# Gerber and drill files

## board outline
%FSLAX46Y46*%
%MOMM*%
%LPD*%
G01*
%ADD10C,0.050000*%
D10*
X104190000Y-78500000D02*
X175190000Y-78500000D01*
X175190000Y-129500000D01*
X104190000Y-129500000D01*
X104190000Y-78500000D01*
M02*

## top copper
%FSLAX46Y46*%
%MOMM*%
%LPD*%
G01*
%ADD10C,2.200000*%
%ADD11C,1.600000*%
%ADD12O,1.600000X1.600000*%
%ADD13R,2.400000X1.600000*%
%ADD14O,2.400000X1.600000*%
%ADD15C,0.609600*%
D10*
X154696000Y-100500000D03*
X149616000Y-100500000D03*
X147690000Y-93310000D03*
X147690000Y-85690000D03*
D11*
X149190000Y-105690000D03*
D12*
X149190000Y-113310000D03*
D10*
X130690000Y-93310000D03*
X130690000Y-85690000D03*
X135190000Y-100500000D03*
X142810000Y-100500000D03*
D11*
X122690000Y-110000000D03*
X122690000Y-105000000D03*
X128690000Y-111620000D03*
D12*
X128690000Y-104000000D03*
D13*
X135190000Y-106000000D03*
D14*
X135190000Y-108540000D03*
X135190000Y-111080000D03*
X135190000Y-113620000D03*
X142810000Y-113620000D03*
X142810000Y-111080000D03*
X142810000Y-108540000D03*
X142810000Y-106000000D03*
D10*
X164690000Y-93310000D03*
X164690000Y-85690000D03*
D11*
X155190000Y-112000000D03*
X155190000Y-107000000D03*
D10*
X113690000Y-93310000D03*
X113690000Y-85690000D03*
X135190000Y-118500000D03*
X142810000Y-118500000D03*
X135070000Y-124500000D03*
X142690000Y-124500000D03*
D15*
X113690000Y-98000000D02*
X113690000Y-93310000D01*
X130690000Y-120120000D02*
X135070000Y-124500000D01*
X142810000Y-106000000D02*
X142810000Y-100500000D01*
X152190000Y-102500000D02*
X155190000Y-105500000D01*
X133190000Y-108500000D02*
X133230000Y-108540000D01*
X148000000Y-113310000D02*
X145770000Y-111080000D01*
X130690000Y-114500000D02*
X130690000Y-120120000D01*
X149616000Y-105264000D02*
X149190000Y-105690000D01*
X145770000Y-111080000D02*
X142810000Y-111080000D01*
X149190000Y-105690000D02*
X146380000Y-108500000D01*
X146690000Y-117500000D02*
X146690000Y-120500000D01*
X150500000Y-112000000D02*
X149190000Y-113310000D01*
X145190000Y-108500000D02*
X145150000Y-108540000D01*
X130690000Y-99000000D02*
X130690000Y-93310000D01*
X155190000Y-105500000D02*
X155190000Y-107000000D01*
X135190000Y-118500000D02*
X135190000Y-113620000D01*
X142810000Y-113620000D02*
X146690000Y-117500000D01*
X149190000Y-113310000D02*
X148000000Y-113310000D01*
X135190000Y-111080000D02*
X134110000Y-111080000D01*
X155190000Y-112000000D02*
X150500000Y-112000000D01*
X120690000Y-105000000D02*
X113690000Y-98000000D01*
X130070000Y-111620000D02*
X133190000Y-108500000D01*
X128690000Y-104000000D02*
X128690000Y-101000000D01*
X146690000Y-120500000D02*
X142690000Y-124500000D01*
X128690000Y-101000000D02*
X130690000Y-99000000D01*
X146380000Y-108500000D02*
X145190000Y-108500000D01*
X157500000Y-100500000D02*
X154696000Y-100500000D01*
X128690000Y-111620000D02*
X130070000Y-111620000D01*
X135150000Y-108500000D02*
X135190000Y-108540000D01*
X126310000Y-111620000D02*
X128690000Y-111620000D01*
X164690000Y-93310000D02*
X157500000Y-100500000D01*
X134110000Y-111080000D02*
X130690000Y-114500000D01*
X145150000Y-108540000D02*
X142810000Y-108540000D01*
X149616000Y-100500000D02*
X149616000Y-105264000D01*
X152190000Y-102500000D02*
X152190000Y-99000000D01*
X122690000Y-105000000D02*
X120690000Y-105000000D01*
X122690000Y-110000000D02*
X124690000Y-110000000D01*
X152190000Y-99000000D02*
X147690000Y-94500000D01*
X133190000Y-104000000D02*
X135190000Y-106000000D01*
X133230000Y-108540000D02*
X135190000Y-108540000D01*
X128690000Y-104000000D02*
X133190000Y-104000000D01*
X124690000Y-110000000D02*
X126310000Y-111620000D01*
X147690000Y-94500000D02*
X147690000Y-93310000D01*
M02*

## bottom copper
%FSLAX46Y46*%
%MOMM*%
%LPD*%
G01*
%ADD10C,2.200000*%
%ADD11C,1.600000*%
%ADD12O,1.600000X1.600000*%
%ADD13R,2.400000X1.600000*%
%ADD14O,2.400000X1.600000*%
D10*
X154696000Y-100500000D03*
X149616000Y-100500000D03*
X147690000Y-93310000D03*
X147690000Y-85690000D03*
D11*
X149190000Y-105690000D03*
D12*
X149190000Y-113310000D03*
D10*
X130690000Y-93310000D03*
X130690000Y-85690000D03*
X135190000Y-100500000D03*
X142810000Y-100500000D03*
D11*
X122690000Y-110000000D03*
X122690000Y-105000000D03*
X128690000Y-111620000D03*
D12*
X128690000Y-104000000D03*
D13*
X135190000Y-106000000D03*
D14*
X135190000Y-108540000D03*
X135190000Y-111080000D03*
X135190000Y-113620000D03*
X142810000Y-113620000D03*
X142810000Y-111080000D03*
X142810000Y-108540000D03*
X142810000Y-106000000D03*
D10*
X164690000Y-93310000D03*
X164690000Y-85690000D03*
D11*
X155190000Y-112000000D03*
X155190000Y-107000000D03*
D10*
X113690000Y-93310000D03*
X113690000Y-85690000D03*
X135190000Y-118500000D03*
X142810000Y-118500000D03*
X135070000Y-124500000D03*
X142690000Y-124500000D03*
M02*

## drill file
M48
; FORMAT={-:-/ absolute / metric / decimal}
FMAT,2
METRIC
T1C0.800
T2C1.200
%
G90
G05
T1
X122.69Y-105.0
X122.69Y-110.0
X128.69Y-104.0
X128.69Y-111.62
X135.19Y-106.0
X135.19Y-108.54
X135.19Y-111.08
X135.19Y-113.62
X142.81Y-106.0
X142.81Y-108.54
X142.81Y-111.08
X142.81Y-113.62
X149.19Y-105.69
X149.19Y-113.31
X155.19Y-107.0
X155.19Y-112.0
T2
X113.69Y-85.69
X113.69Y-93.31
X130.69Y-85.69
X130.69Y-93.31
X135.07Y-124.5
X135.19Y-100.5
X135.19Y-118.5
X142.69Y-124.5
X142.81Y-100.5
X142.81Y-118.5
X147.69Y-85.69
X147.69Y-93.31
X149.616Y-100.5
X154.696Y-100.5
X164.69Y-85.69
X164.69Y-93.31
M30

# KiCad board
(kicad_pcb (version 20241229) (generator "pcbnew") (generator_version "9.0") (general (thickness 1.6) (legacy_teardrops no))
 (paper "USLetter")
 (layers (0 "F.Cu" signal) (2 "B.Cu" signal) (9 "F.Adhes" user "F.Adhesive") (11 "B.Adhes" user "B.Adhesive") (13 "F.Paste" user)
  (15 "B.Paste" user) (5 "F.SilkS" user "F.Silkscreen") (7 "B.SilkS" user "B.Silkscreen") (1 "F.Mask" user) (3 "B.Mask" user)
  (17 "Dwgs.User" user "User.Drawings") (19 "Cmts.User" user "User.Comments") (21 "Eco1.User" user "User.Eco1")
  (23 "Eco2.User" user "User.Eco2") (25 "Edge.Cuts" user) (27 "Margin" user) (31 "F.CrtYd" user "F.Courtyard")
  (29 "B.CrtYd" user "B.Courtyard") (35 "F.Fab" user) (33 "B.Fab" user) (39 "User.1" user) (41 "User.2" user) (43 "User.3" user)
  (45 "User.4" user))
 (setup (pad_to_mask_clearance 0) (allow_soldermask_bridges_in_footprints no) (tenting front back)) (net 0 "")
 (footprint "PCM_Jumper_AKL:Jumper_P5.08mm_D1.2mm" (layer "F.Cu") (at 154.696 100.5 180)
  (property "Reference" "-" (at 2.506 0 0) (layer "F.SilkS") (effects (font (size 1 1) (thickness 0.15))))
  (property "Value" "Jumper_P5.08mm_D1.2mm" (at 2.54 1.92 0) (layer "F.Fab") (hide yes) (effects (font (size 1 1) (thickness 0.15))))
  (pad "1" thru_hole circle (at 0 0 180) (size 2.2 2.2) (drill 1.2) (layers "*.Cu" "*.Mask") (remove_unused_layers no))
  (pad "2" thru_hole circle (at 5.08 0 180) (size 2.2 2.2) (drill 1.2) (layers "*.Cu" "*.Mask") (remove_unused_layers no)))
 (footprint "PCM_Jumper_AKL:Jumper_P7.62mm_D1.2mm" (layer "F.Cu") (at 147.69 93.31 90)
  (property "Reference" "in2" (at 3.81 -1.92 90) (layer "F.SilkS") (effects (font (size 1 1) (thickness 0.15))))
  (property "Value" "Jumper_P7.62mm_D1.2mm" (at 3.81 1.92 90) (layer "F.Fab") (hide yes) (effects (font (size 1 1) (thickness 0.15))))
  (pad "1" thru_hole circle (at 0 0 90) (size 2.2 2.2) (drill 1.2) (layers "*.Cu" "*.Mask") (remove_unused_layers no))
  (pad "2" thru_hole circle (at 7.62 0 90) (size 2.2 2.2) (drill 1.2) (layers "*.Cu" "*.Mask") (remove_unused_layers no)))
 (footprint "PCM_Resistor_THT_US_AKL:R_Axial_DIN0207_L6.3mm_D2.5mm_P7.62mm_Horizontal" (layer "F.Cu") (at 149.19 105.69 -90)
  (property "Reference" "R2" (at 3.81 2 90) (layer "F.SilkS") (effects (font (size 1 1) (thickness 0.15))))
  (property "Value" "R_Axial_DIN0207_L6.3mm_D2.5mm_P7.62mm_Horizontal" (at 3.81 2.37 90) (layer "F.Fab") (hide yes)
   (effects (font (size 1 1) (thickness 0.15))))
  (pad "1" thru_hole circle (at 0 0 270) (size 1.6 1.6) (drill 0.8) (layers "*.Cu" "*.Mask") (remove_unused_layers no))
  (pad "2" thru_hole oval (at 7.62 0 270) (size 1.6 1.6) (drill 0.8) (layers "*.Cu" "*.Mask") (remove_unused_layers no)))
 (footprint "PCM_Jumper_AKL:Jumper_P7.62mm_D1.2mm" (layer "F.Cu") (at 130.69 93.31 90)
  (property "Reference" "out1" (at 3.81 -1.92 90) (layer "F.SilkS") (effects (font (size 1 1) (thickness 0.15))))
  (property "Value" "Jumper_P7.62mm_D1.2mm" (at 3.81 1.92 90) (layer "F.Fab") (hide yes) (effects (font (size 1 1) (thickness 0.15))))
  (pad "1" thru_hole circle (at 0 0 90) (size 2.2 2.2) (drill 1.2) (layers "*.Cu" "*.Mask") (remove_unused_layers no))
  (pad "2" thru_hole circle (at 7.62 0 90) (size 2.2 2.2) (drill 1.2) (layers "*.Cu" "*.Mask") (remove_unused_layers no)))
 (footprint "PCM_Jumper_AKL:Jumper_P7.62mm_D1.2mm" (layer "F.Cu") (at 135.19 100.5)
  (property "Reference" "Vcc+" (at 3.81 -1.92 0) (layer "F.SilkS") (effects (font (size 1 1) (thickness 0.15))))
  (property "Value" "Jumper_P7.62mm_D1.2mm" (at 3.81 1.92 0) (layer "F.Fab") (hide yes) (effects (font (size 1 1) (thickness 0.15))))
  (pad "1" thru_hole circle (at 0 0) (size 2.2 2.2) (drill 1.2) (layers "*.Cu" "*.Mask") (remove_unused_layers no))
  (pad "2" thru_hole circle (at 7.62 0) (size 2.2 2.2) (drill 1.2) (layers "*.Cu" "*.Mask") (remove_unused_layers no)))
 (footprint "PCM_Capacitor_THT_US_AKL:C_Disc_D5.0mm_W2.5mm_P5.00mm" (layer "F.Cu") (at 122.69 110 90)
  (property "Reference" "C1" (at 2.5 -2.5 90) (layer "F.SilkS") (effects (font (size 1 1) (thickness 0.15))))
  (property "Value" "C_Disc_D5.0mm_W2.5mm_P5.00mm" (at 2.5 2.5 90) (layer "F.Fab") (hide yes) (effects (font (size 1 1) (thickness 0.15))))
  (pad "1" thru_hole circle (at 0 0 90) (size 1.6 1.6) (drill 0.8) (layers "*.Cu" "*.Mask") (remove_unused_layers no))
  (pad "2" thru_hole circle (at 5 0 90) (size 1.6 1.6) (drill 0.8) (layers "*.Cu" "*.Mask") (remove_unused_layers no)))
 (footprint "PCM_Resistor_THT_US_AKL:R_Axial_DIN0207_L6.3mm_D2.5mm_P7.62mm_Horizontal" (layer "F.Cu") (at 128.69 111.62 90)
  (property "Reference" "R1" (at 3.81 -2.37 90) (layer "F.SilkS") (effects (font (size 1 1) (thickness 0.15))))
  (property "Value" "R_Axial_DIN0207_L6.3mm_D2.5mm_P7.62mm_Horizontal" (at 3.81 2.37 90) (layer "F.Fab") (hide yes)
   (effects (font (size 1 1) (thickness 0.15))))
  (pad "1" thru_hole circle (at 0 0 90) (size 1.6 1.6) (drill 0.8) (layers "*.Cu" "*.Mask") (remove_unused_layers no))
  (pad "2" thru_hole oval (at 7.62 0 90) (size 1.6 1.6) (drill 0.8) (layers "*.Cu" "*.Mask") (remove_unused_layers no)))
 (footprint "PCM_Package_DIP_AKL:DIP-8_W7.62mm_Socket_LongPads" (layer "F.Cu") (at 135.19 106)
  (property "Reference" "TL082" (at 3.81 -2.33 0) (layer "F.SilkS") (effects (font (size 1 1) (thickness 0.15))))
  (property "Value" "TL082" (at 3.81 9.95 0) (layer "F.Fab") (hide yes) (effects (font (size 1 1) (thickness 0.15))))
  (pad "1" thru_hole rect (at 0 0) (size 2.4 1.6) (drill 0.8) (layers "*.Cu" "*.Mask") (remove_unused_layers no))
  (pad "2" thru_hole oval (at 0 2.54) (size 2.4 1.6) (drill 0.8) (layers "*.Cu" "*.Mask") (remove_unused_layers no))
  (pad "3" thru_hole oval (at 0 5.08) (size 2.4 1.6) (drill 0.8) (layers "*.Cu" "*.Mask") (remove_unused_layers no))
  (pad "4" thru_hole oval (at 0 7.62) (size 2.4 1.6) (drill 0.8) (layers "*.Cu" "*.Mask") (remove_unused_layers no))
  (pad "5" thru_hole oval (at 7.62 7.62) (size 2.4 1.6) (drill 0.8) (layers "*.Cu" "*.Mask") (remove_unused_layers no))
  (pad "6" thru_hole oval (at 7.62 5.08) (size 2.4 1.6) (drill 0.8) (layers "*.Cu" "*.Mask") (remove_unused_layers no))
  (pad "7" thru_hole oval (at 7.62 2.54) (size 2.4 1.6) (drill 0.8) (layers "*.Cu" "*.Mask") (remove_unused_layers no))
  (pad "8" thru_hole oval (at 7.62 0) (size 2.4 1.6) (drill 0.8) (layers "*.Cu" "*.Mask") (remove_unused_layers no)))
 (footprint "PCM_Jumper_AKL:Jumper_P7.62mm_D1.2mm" (layer "F.Cu") (at 164.69 93.31 90)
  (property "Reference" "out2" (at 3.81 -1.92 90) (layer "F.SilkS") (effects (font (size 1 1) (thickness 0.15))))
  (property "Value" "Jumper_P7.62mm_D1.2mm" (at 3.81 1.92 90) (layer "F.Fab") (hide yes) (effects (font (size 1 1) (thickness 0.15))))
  (pad "1" thru_hole circle (at 0 0 90) (size 2.2 2.2) (drill 1.2) (layers "*.Cu" "*.Mask") (remove_unused_layers no))
  (pad "2" thru_hole circle (at 7.62 0 90) (size 2.2 2.2) (drill 1.2) (layers "*.Cu" "*.Mask") (remove_unused_layers no)))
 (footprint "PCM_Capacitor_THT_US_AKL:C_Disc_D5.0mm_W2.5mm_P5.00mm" (layer "F.Cu") (at 155.19 112 90)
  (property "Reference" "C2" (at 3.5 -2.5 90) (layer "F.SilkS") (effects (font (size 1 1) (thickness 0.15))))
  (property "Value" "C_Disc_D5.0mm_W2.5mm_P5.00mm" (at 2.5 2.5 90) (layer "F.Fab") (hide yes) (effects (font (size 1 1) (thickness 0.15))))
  (pad "1" thru_hole circle (at 0 0 90) (size 1.6 1.6) (drill 0.8) (layers "*.Cu" "*.Mask") (remove_unused_layers no))
  (pad "2" thru_hole circle (at 5 0 90) (size 1.6 1.6) (drill 0.8) (layers "*.Cu" "*.Mask") (remove_unused_layers no)))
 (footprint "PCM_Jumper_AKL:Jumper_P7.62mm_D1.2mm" (layer "F.Cu") (at 113.69 93.31 90)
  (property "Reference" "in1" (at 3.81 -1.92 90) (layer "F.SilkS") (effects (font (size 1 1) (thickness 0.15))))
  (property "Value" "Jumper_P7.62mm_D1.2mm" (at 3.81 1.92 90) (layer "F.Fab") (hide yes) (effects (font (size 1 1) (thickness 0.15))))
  (pad "1" thru_hole circle (at 0 0 90) (size 2.2 2.2) (drill 1.2) (layers "*.Cu" "*.Mask") (remove_unused_layers no))
  (pad "2" thru_hole circle (at 7.62 0 90) (size 2.2 2.2) (drill 1.2) (layers "*.Cu" "*.Mask") (remove_unused_layers no)))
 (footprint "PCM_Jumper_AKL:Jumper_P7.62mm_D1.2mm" (layer "F.Cu") (at 135.19 118.5)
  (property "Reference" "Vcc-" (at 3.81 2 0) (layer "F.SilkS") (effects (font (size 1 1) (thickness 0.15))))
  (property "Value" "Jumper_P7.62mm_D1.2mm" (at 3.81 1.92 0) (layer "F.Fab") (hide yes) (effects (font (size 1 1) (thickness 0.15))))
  (pad "1" thru_hole circle (at 0 0) (size 2.2 2.2) (drill 1.2) (layers "*.Cu" "*.Mask") (remove_unused_layers no))
  (pad "2" thru_hole circle (at 7.62 0) (size 2.2 2.2) (drill 1.2) (layers "*.Cu" "*.Mask") (remove_unused_layers no)))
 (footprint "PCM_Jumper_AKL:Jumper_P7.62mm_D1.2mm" (layer "F.Cu") (at 135.07 124.5)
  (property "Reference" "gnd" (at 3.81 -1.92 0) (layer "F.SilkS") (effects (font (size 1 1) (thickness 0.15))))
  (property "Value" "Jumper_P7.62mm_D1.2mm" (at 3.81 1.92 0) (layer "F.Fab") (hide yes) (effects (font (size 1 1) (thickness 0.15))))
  (pad "1" thru_hole circle (at 0 0) (size 2.2 2.2) (drill 1.2) (layers "*.Cu" "*.Mask") (remove_unused_layers no))
  (pad "2" thru_hole circle (at 7.62 0) (size 2.2 2.2) (drill 1.2) (layers "*.Cu" "*.Mask") (remove_unused_layers no)))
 (gr_rect (start 104.19 78.5) (end 175.19 129.5) (stroke (width 0.05) (type default)) (fill no) (layer "Edge.Cuts"))
 (segment (start 113.69 98) (end 113.69 93.31) (width 0.6096) (layer "F.Cu") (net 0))
 (segment (start 130.69 120.12) (end 135.07 124.5) (width 0.6096) (layer "F.Cu") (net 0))
 (segment (start 142.81 106) (end 142.81 100.5) (width 0.6096) (layer "F.Cu") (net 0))
 (segment (start 152.19 102.5) (end 155.19 105.5) (width 0.6096) (layer "F.Cu") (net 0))
 (segment (start 133.19 108.5) (end 133.23 108.54) (width 0.6096) (layer "F.Cu") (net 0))
 (segment (start 148 113.31) (end 145.77 111.08) (width 0.6096) (layer "F.Cu") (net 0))
 (segment (start 130.69 114.5) (end 130.69 120.12) (width 0.6096) (layer "F.Cu") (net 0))
 (segment (start 149.616 105.264) (end 149.19 105.69) (width 0.6096) (layer "F.Cu") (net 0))
 (segment (start 145.77 111.08) (end 142.81 111.08) (width 0.6096) (layer "F.Cu") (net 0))
 (segment (start 149.19 105.69) (end 146.38 108.5) (width 0.6096) (layer "F.Cu") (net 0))
 (segment (start 146.69 117.5) (end 146.69 120.5) (width 0.6096) (layer "F.Cu") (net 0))
 (segment (start 150.5 112) (end 149.19 113.31) (width 0.6096) (layer "F.Cu") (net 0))
 (segment (start 145.19 108.5) (end 145.15 108.54) (width 0.6096) (layer "F.Cu") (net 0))
 (segment (start 130.69 99) (end 130.69 93.31) (width 0.6096) (layer "F.Cu") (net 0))
 (segment (start 155.19 105.5) (end 155.19 107) (width 0.6096) (layer "F.Cu") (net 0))
 (segment (start 135.19 118.5) (end 135.19 113.62) (width 0.6096) (layer "F.Cu") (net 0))
 (segment (start 142.81 113.62) (end 146.69 117.5) (width 0.6096) (layer "F.Cu") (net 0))
 (segment (start 149.19 113.31) (end 148 113.31) (width 0.6096) (layer "F.Cu") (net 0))
 (segment (start 135.19 111.08) (end 134.11 111.08) (width 0.6096) (layer "F.Cu") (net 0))
 (segment (start 155.19 112) (end 150.5 112) (width 0.6096) (layer "F.Cu") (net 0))
 (segment (start 120.69 105) (end 113.69 98) (width 0.6096) (layer "F.Cu") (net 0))
 (segment (start 130.07 111.62) (end 133.19 108.5) (width 0.6096) (layer "F.Cu") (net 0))
 (segment (start 128.69 104) (end 128.69 101) (width 0.6096) (layer "F.Cu") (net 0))
 (segment (start 146.69 120.5) (end 142.69 124.5) (width 0.6096) (layer "F.Cu") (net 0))
 (segment (start 128.69 101) (end 130.69 99) (width 0.6096) (layer "F.Cu") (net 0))
 (segment (start 146.38 108.5) (end 145.19 108.5) (width 0.6096) (layer "F.Cu") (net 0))
 (segment (start 157.5 100.5) (end 154.696 100.5) (width 0.6096) (layer "F.Cu") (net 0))
 (segment (start 128.69 111.62) (end 130.07 111.62) (width 0.6096) (layer "F.Cu") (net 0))
 (segment (start 135.15 108.5) (end 135.19 108.54) (width 0.6096) (layer "F.Cu") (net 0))
 (segment (start 126.31 111.62) (end 128.69 111.62) (width 0.6096) (layer "F.Cu") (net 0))
 (segment (start 164.69 93.31) (end 157.5 100.5) (width 0.6096) (layer "F.Cu") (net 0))
 (segment (start 134.11 111.08) (end 130.69 114.5) (width 0.6096) (layer "F.Cu") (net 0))
 (segment (start 145.15 108.54) (end 142.81 108.54) (width 0.6096) (layer "F.Cu") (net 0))
 (segment (start 149.616 100.5) (end 149.616 105.264) (width 0.6096) (layer "F.Cu") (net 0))
 (segment (start 152.19 102.5) (end 152.19 99) (width 0.6096) (layer "F.Cu") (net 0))
 (segment (start 122.69 105) (end 120.69 105) (width 0.6096) (layer "F.Cu") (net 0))
 (segment (start 122.69 110) (end 124.69 110) (width 0.6096) (layer "F.Cu") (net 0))
 (segment (start 152.19 99) (end 147.69 94.5) (width 0.6096) (layer "F.Cu") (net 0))
 (segment (start 133.19 104) (end 135.19 106) (width 0.6096) (layer "F.Cu") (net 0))
 (segment (start 133.23 108.54) (end 135.19 108.54) (width 0.6096) (layer "F.Cu") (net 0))
 (segment (start 128.69 104) (end 133.19 104) (width 0.6096) (layer "F.Cu") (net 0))
 (segment (start 124.69 110) (end 126.31 111.62) (width 0.6096) (layer "F.Cu") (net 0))
 (segment (start 147.69 94.5) (end 147.69 93.31) (width 0.6096) (layer "F.Cu") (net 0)))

